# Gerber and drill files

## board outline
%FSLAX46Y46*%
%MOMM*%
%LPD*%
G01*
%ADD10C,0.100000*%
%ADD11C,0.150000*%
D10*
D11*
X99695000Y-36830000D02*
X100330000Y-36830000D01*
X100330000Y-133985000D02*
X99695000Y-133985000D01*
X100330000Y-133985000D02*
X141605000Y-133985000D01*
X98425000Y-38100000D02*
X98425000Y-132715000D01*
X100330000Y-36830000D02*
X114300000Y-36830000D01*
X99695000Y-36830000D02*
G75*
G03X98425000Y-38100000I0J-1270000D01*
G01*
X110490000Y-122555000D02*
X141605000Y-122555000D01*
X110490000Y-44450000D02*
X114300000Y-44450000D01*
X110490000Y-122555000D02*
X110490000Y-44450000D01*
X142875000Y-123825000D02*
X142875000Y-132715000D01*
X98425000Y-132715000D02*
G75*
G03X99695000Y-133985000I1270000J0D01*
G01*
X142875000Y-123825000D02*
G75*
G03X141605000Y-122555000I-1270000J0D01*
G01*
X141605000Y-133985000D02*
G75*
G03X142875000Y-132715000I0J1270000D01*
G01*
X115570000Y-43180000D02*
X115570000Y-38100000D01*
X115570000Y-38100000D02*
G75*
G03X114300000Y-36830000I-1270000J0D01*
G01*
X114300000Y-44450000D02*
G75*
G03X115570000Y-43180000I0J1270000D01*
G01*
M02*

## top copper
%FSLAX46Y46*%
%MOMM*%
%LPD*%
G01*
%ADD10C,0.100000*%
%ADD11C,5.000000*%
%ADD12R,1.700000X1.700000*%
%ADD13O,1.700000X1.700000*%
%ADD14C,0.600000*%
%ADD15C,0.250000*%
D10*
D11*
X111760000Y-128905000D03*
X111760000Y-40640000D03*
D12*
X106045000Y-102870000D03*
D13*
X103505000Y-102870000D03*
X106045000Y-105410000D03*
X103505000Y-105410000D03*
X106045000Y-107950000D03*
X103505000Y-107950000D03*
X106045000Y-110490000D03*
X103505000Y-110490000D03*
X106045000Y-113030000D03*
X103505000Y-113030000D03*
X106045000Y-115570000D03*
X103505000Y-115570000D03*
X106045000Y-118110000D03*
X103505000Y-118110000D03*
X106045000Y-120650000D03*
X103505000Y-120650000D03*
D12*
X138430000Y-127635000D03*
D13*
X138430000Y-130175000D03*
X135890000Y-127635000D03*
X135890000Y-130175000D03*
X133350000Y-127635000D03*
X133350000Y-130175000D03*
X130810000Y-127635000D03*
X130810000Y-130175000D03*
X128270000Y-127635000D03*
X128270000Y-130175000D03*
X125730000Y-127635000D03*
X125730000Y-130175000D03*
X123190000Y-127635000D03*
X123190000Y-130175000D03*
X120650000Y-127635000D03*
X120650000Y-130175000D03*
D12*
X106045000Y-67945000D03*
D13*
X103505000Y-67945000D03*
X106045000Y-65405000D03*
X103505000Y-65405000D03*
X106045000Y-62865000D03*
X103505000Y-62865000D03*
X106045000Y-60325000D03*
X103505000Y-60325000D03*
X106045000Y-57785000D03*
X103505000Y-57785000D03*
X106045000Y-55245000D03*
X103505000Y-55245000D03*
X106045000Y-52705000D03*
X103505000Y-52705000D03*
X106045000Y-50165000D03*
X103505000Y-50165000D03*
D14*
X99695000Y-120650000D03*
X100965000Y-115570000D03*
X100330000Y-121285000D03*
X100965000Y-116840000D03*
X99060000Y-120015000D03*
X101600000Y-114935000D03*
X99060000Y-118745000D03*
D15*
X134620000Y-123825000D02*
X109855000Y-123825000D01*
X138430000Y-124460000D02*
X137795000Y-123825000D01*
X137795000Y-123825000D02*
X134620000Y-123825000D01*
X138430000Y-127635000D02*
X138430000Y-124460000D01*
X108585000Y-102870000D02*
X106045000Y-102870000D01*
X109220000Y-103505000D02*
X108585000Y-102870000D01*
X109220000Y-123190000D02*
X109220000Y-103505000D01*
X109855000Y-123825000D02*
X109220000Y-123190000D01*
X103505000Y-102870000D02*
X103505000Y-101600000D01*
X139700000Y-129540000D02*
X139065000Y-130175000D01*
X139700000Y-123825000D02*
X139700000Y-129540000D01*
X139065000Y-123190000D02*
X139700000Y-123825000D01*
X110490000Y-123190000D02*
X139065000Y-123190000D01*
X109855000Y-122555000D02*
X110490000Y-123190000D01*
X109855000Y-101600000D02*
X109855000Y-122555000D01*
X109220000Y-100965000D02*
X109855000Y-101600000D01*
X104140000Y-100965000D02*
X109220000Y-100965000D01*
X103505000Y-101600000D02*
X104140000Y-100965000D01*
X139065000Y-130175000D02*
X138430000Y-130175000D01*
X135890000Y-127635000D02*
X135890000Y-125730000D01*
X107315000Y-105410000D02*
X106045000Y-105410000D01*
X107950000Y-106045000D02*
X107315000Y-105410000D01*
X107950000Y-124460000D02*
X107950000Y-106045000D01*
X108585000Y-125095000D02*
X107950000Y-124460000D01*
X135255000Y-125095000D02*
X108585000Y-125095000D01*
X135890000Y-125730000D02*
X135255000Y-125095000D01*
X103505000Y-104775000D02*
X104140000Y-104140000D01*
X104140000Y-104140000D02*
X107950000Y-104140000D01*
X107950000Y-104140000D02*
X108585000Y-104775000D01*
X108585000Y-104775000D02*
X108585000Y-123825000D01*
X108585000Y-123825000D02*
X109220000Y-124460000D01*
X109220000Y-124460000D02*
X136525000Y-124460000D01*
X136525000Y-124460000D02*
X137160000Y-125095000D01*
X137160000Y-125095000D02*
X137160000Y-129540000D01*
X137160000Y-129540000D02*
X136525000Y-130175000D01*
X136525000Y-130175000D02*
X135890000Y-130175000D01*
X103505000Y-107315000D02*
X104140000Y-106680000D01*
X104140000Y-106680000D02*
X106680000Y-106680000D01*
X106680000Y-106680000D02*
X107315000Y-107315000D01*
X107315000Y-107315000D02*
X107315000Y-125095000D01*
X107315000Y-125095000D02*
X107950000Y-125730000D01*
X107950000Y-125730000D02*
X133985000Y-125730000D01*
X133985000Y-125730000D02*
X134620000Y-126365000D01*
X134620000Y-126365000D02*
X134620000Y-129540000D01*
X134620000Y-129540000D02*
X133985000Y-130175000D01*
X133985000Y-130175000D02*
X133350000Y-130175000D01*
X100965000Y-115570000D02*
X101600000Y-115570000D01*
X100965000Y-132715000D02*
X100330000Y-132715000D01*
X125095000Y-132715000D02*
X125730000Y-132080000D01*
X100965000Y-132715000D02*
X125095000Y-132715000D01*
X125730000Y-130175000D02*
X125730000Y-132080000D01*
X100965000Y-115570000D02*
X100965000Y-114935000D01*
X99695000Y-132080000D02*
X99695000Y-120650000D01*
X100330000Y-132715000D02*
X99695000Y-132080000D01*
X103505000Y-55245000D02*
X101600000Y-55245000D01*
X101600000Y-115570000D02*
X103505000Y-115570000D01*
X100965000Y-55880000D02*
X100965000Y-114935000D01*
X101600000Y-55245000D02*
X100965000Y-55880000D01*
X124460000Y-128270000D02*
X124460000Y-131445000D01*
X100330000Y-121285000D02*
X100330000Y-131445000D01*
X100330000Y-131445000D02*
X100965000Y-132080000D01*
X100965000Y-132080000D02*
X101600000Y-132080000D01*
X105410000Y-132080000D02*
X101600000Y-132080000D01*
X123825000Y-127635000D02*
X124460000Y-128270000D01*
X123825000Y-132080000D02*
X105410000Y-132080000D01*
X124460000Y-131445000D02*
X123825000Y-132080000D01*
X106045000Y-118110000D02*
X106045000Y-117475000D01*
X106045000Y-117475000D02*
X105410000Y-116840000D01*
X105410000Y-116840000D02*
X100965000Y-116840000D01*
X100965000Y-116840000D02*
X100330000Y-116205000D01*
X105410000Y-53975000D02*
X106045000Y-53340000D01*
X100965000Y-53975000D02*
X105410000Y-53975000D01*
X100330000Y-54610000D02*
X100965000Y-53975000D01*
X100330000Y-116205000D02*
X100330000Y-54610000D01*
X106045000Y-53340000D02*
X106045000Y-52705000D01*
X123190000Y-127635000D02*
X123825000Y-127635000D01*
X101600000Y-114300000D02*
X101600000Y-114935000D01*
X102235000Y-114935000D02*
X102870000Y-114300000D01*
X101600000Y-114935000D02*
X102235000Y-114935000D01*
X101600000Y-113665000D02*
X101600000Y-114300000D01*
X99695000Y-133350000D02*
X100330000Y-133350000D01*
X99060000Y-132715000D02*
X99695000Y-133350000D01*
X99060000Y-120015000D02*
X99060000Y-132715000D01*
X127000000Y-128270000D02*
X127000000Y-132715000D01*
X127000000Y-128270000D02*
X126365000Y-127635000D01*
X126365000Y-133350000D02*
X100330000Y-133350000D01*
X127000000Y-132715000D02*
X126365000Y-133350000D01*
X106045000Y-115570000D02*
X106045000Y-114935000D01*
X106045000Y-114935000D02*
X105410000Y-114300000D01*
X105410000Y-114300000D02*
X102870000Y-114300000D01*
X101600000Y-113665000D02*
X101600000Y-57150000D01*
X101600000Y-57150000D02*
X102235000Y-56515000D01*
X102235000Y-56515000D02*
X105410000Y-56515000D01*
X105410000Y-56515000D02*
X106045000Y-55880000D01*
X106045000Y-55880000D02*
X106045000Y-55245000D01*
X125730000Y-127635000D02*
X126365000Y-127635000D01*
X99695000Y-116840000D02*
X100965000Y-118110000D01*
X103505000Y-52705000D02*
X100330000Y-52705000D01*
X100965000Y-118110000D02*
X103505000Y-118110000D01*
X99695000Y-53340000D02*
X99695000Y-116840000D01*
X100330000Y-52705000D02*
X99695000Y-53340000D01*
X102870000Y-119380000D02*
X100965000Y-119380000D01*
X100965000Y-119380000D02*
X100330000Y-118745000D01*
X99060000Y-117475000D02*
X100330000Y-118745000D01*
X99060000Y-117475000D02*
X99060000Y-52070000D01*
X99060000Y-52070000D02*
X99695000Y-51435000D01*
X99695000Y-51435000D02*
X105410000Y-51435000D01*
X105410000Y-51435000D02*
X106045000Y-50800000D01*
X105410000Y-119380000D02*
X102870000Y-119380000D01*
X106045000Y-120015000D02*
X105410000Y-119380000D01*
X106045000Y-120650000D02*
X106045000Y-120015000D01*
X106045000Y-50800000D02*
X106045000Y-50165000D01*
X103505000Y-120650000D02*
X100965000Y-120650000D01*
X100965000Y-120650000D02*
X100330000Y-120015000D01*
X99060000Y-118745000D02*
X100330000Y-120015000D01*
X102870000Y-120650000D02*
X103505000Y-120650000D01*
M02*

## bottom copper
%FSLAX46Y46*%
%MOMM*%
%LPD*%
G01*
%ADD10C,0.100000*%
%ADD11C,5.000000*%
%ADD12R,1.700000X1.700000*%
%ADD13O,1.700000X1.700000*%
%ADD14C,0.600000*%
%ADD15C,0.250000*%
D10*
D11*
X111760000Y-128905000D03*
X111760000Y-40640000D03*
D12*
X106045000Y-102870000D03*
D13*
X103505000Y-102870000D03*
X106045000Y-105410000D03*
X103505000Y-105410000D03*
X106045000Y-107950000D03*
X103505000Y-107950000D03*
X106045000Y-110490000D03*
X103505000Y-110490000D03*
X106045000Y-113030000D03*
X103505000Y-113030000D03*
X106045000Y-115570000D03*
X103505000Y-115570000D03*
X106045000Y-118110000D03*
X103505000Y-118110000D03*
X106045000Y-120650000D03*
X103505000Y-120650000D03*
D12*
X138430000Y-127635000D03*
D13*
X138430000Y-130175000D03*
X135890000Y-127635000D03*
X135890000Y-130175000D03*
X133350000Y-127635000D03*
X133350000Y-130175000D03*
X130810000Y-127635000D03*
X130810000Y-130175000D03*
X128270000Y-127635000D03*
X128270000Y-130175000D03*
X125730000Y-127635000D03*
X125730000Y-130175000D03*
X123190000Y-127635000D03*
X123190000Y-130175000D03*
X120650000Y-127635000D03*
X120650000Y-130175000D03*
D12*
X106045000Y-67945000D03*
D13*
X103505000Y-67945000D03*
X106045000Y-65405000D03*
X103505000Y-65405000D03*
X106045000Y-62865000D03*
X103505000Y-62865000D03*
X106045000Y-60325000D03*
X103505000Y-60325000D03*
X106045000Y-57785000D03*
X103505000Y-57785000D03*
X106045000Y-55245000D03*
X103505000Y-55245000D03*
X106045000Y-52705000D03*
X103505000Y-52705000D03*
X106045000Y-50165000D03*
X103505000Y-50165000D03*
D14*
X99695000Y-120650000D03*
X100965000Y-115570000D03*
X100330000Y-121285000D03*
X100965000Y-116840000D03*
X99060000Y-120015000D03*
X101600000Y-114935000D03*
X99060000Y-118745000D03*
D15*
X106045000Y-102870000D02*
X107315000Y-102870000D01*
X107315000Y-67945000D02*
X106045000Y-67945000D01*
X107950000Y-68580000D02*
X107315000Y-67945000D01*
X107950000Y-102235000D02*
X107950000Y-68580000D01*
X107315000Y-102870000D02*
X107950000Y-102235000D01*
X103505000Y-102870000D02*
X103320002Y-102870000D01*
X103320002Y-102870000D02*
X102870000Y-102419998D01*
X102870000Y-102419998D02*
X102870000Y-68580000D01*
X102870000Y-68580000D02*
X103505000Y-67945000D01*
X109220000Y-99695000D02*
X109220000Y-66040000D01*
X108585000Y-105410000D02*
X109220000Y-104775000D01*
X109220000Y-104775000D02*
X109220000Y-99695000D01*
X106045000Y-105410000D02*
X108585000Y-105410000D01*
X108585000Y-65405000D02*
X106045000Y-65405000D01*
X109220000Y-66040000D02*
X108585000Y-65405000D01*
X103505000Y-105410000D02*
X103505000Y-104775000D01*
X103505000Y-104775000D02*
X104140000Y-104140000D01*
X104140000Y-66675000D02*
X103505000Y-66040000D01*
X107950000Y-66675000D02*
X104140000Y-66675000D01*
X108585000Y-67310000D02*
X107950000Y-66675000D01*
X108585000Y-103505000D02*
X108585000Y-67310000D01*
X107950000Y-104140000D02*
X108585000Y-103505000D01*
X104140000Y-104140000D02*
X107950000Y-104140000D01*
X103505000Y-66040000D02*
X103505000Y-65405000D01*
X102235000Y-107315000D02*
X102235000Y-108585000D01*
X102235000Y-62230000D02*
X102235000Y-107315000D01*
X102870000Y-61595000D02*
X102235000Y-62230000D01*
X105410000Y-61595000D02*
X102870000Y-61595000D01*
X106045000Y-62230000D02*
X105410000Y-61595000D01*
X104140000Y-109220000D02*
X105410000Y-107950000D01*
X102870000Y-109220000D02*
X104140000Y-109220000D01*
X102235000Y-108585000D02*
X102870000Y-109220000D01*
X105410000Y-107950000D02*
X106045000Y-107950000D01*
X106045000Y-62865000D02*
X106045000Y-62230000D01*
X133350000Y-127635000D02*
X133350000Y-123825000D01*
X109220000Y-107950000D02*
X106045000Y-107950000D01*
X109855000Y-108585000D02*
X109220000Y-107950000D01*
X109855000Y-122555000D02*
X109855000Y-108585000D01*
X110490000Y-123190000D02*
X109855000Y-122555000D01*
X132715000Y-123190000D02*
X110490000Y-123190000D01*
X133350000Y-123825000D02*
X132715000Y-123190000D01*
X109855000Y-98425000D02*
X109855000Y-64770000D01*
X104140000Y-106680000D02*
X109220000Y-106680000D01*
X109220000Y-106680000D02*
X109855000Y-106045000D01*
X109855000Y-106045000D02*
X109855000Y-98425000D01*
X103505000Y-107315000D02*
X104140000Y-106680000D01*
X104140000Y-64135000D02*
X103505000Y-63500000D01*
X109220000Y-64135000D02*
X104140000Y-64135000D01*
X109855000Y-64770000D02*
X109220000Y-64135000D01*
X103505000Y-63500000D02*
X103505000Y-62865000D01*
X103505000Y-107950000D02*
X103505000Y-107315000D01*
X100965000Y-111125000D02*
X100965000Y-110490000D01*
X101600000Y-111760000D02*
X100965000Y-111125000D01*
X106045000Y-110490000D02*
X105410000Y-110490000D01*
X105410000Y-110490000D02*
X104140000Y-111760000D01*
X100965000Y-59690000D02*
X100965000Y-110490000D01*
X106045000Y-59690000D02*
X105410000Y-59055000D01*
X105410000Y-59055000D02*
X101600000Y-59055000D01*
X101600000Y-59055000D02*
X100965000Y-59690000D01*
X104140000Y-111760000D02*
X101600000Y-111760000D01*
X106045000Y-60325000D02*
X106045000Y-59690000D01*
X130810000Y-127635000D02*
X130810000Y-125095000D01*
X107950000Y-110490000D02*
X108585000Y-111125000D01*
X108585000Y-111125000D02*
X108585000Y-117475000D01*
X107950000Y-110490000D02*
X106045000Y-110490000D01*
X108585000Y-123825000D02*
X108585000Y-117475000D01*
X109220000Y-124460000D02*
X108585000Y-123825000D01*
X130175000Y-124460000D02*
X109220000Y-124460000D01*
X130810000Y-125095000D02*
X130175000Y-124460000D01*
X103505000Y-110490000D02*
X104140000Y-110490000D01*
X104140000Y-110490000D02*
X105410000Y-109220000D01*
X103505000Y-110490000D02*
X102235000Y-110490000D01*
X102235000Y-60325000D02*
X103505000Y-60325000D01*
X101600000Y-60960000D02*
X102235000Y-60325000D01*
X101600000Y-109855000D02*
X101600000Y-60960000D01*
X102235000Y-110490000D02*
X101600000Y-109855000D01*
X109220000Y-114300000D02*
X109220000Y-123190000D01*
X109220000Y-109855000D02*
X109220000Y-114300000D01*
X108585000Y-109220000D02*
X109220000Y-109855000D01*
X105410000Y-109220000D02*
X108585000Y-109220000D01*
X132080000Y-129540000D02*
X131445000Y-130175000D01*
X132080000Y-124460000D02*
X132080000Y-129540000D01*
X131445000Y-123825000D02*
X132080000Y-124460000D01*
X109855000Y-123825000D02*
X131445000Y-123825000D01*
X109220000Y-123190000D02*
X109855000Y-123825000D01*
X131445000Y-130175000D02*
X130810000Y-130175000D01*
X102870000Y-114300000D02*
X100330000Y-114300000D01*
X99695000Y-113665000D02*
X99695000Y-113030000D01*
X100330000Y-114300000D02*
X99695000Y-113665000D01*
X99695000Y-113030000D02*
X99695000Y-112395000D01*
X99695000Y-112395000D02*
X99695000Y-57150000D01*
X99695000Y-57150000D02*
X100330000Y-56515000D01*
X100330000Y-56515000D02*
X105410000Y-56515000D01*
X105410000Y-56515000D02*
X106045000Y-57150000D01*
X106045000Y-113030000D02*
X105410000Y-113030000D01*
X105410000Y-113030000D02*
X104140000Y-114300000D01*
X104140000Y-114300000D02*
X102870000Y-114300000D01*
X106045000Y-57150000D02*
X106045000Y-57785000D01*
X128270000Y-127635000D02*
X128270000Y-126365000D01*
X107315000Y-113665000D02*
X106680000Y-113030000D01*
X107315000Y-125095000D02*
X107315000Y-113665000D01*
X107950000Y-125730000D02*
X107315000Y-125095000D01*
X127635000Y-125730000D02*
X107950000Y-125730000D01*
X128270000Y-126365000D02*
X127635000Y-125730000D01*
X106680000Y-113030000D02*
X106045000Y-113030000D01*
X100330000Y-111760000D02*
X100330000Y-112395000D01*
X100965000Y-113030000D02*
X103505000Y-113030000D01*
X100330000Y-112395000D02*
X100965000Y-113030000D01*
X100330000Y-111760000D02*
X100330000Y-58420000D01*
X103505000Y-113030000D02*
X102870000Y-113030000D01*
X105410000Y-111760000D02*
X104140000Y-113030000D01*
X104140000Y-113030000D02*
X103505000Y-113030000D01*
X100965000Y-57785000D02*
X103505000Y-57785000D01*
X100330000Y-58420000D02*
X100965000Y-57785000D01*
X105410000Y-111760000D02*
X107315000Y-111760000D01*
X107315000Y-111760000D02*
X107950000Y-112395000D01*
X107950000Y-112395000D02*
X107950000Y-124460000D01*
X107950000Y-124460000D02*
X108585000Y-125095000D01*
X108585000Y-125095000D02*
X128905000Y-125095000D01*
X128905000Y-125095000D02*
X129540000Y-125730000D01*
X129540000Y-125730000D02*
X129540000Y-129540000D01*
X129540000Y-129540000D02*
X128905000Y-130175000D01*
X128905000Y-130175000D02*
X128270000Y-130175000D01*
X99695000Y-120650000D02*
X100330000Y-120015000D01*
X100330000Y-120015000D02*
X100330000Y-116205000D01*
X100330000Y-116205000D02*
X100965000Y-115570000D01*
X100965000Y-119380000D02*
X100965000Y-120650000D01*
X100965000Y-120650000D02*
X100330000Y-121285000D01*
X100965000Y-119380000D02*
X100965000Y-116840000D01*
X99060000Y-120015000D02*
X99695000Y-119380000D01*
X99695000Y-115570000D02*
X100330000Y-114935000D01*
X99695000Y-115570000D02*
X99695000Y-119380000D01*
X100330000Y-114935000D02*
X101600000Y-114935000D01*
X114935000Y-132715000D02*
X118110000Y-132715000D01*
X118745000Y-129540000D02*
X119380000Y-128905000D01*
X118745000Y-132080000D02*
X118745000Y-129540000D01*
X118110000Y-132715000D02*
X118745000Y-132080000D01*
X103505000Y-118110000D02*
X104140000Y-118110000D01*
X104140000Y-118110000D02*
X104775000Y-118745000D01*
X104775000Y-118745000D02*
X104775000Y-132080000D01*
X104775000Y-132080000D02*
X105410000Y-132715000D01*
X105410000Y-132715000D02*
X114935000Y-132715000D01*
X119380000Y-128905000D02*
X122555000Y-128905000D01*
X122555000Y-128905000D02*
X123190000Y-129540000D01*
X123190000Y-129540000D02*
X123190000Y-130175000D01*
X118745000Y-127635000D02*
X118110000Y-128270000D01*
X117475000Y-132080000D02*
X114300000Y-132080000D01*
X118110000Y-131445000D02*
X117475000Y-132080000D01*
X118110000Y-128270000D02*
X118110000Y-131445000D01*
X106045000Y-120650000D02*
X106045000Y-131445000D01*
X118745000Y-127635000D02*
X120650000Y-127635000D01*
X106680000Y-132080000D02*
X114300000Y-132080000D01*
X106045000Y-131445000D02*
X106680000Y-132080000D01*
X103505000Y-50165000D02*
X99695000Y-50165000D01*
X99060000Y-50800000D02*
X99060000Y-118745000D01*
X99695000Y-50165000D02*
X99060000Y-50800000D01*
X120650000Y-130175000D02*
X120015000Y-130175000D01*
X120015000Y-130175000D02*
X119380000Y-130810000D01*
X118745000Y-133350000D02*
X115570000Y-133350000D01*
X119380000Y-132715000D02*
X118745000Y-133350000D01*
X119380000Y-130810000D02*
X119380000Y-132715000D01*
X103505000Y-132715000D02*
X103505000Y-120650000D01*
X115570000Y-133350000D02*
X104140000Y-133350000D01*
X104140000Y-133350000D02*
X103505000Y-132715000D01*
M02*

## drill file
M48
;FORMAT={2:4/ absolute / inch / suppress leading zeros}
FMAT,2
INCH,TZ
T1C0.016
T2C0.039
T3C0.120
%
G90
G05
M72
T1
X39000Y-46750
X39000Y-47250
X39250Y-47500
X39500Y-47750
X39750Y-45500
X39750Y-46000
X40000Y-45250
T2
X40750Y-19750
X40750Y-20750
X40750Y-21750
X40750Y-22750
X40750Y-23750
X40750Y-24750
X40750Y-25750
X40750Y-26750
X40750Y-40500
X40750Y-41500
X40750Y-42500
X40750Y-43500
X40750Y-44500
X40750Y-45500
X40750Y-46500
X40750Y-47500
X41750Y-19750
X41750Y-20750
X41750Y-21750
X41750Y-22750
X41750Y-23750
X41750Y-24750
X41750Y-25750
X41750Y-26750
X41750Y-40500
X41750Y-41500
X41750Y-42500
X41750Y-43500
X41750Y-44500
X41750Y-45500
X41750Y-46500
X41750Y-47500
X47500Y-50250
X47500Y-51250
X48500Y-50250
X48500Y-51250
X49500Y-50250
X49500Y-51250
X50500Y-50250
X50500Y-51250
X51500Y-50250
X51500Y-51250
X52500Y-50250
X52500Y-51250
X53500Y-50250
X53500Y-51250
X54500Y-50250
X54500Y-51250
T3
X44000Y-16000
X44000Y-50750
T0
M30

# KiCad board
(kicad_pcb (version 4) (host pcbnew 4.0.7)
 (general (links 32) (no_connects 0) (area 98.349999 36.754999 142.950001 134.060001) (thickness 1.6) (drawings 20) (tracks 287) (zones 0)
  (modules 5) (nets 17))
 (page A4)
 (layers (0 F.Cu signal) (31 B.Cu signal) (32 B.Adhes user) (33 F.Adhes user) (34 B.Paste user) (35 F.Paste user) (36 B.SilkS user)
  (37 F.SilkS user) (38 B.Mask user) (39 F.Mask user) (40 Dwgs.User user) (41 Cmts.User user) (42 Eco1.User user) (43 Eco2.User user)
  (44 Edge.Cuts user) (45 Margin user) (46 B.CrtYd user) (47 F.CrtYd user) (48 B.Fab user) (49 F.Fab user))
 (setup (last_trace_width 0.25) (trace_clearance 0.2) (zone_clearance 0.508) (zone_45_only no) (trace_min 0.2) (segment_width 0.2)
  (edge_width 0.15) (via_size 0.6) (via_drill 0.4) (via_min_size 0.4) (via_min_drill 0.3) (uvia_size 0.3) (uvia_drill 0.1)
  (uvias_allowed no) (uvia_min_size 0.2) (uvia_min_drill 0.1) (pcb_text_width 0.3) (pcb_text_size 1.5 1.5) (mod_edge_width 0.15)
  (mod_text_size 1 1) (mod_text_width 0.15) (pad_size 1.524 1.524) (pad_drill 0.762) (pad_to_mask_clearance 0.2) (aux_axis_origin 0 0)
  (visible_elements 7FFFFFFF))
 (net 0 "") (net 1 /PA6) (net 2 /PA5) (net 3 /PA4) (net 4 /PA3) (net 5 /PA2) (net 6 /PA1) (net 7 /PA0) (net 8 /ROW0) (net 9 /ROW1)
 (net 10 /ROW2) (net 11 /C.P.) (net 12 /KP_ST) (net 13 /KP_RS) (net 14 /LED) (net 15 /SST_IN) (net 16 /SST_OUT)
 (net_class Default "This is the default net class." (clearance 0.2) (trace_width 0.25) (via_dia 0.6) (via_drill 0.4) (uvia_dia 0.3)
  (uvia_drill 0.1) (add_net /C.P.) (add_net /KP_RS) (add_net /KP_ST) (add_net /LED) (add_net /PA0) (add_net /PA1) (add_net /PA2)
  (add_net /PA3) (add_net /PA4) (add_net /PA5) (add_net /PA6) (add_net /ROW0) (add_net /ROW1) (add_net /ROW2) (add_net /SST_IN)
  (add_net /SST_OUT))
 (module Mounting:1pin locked (layer F.Cu) (at 111.76 128.905)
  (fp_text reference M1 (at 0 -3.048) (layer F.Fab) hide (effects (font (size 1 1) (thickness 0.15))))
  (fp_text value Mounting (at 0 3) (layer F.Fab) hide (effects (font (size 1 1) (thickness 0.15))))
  (pad 1 thru_hole circle (at 0 0) (size 5 5) (drill 3.048) (layers *.Cu *.Mask)))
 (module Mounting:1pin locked (layer F.Cu) (at 111.76 40.64)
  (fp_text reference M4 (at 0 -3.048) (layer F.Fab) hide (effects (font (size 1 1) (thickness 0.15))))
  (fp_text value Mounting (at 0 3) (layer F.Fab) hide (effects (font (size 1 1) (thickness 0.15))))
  (pad 1 thru_hole circle (at 0 0) (size 5 5) (drill 3.048) (layers *.Cu *.Mask)))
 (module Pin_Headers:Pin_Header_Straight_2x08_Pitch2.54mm (layer B.Cu) (at 106.045 102.87 180)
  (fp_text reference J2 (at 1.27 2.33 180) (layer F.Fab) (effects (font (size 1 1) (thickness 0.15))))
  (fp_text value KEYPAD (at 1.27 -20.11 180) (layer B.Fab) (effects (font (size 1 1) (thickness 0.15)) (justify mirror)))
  (pad 1 thru_hole rect (at 0 0 180) (size 1.7 1.7) (drill 1) (layers *.Cu *.Mask) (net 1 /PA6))
  (pad 2 thru_hole oval (at 2.54 0 180) (size 1.7 1.7) (drill 1) (layers *.Cu *.Mask) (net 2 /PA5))
  (pad 3 thru_hole oval (at 0 -2.54 180) (size 1.7 1.7) (drill 1) (layers *.Cu *.Mask) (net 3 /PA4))
  (pad 4 thru_hole oval (at 2.54 -2.54 180) (size 1.7 1.7) (drill 1) (layers *.Cu *.Mask) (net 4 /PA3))
  (pad 5 thru_hole oval (at 0 -5.08 180) (size 1.7 1.7) (drill 1) (layers *.Cu *.Mask) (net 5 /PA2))
  (pad 6 thru_hole oval (at 2.54 -5.08 180) (size 1.7 1.7) (drill 1) (layers *.Cu *.Mask) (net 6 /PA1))
  (pad 7 thru_hole oval (at 0 -7.62 180) (size 1.7 1.7) (drill 1) (layers *.Cu *.Mask) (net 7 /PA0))
  (pad 8 thru_hole oval (at 2.54 -7.62 180) (size 1.7 1.7) (drill 1) (layers *.Cu *.Mask) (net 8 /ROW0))
  (pad 9 thru_hole oval (at 0 -10.16 180) (size 1.7 1.7) (drill 1) (layers *.Cu *.Mask) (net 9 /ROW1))
  (pad 10 thru_hole oval (at 2.54 -10.16 180) (size 1.7 1.7) (drill 1) (layers *.Cu *.Mask) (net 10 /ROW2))
  (pad 11 thru_hole oval (at 0 -12.7 180) (size 1.7 1.7) (drill 1) (layers *.Cu *.Mask) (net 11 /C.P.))
  (pad 12 thru_hole oval (at 2.54 -12.7 180) (size 1.7 1.7) (drill 1) (layers *.Cu *.Mask) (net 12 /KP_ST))
  (pad 13 thru_hole oval (at 0 -15.24 180) (size 1.7 1.7) (drill 1) (layers *.Cu *.Mask) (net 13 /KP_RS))
  (pad 14 thru_hole oval (at 2.54 -15.24 180) (size 1.7 1.7) (drill 1) (layers *.Cu *.Mask) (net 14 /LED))
  (pad 15 thru_hole oval (at 0 -17.78 180) (size 1.7 1.7) (drill 1) (layers *.Cu *.Mask) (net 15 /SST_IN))
  (pad 16 thru_hole oval (at 2.54 -17.78 180) (size 1.7 1.7) (drill 1) (layers *.Cu *.Mask) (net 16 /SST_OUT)))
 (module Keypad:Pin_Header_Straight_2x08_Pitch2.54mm (layer F.Cu) (at 138.43 127.635 270)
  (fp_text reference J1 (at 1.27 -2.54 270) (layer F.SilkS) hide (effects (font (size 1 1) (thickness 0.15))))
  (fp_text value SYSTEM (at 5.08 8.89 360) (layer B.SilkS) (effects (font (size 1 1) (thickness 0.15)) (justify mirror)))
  (pad 1 thru_hole rect (at 0 0 270) (size 1.7 1.7) (drill 1) (layers *.Cu *.Mask) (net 1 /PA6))
  (pad 2 thru_hole oval (at 2.54 0 270) (size 1.7 1.7) (drill 1) (layers *.Cu *.Mask) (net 2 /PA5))
  (pad 3 thru_hole oval (at 0 2.54 270) (size 1.7 1.7) (drill 1) (layers *.Cu *.Mask) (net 3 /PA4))
  (pad 4 thru_hole oval (at 2.54 2.54 270) (size 1.7 1.7) (drill 1) (layers *.Cu *.Mask) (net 4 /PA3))
  (pad 5 thru_hole oval (at 0 5.08 270) (size 1.7 1.7) (drill 1) (layers *.Cu *.Mask) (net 5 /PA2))
  (pad 6 thru_hole oval (at 2.54 5.08 270) (size 1.7 1.7) (drill 1) (layers *.Cu *.Mask) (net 6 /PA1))
  (pad 7 thru_hole oval (at 0 7.62 270) (size 1.7 1.7) (drill 1) (layers *.Cu *.Mask) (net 7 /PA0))
  (pad 8 thru_hole oval (at 2.54 7.62 270) (size 1.7 1.7) (drill 1) (layers *.Cu *.Mask) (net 8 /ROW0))
  (pad 9 thru_hole oval (at 0 10.16 270) (size 1.7 1.7) (drill 1) (layers *.Cu *.Mask) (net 9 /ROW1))
  (pad 10 thru_hole oval (at 2.54 10.16 270) (size 1.7 1.7) (drill 1) (layers *.Cu *.Mask) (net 10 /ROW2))
  (pad 11 thru_hole oval (at 0 12.7 270) (size 1.7 1.7) (drill 1) (layers *.Cu *.Mask) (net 11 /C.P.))
  (pad 12 thru_hole oval (at 2.54 12.7 270) (size 1.7 1.7) (drill 1) (layers *.Cu *.Mask) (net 12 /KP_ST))
  (pad 13 thru_hole oval (at 0 15.24 270) (size 1.7 1.7) (drill 1) (layers *.Cu *.Mask) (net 13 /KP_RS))
  (pad 14 thru_hole oval (at 2.54 15.24 270) (size 1.7 1.7) (drill 1) (layers *.Cu *.Mask) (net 14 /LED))
  (pad 15 thru_hole oval (at 0 17.78 270) (size 1.7 1.7) (drill 1) (layers *.Cu *.Mask) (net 15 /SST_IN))
  (pad 16 thru_hole oval (at 2.54 17.78 270) (size 1.7 1.7) (drill 1) (layers *.Cu *.Mask) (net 16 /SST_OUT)))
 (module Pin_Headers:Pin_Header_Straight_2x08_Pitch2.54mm (layer F.Cu) (at 106.045 67.945 180)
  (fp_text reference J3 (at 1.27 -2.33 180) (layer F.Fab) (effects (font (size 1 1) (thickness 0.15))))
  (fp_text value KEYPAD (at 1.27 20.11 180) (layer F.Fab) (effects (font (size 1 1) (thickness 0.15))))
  (pad 1 thru_hole rect (at 0 0 180) (size 1.7 1.7) (drill 1) (layers *.Cu *.Mask) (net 1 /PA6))
  (pad 2 thru_hole oval (at 2.54 0 180) (size 1.7 1.7) (drill 1) (layers *.Cu *.Mask) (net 2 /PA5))
  (pad 3 thru_hole oval (at 0 2.54 180) (size 1.7 1.7) (drill 1) (layers *.Cu *.Mask) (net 3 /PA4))
  (pad 4 thru_hole oval (at 2.54 2.54 180) (size 1.7 1.7) (drill 1) (layers *.Cu *.Mask) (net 4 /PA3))
  (pad 5 thru_hole oval (at 0 5.08 180) (size 1.7 1.7) (drill 1) (layers *.Cu *.Mask) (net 5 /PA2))
  (pad 6 thru_hole oval (at 2.54 5.08 180) (size 1.7 1.7) (drill 1) (layers *.Cu *.Mask) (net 6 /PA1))
  (pad 7 thru_hole oval (at 0 7.62 180) (size 1.7 1.7) (drill 1) (layers *.Cu *.Mask) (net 7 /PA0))
  (pad 8 thru_hole oval (at 2.54 7.62 180) (size 1.7 1.7) (drill 1) (layers *.Cu *.Mask) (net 8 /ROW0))
  (pad 9 thru_hole oval (at 0 10.16 180) (size 1.7 1.7) (drill 1) (layers *.Cu *.Mask) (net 9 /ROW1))
  (pad 10 thru_hole oval (at 2.54 10.16 180) (size 1.7 1.7) (drill 1) (layers *.Cu *.Mask) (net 10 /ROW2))
  (pad 11 thru_hole oval (at 0 12.7 180) (size 1.7 1.7) (drill 1) (layers *.Cu *.Mask) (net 11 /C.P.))
  (pad 12 thru_hole oval (at 2.54 12.7 180) (size 1.7 1.7) (drill 1) (layers *.Cu *.Mask) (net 12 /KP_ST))
  (pad 13 thru_hole oval (at 0 15.24 180) (size 1.7 1.7) (drill 1) (layers *.Cu *.Mask) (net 13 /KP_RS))
  (pad 14 thru_hole oval (at 2.54 15.24 180) (size 1.7 1.7) (drill 1) (layers *.Cu *.Mask) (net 14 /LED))
  (pad 15 thru_hole oval (at 0 17.78 180) (size 1.7 1.7) (drill 1) (layers *.Cu *.Mask) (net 15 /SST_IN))
  (pad 16 thru_hole oval (at 2.54 17.78 180) (size 1.7 1.7) (drill 1) (layers *.Cu *.Mask) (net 16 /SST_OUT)))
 (gr_line (start 99.695 36.83) (end 100.33 36.83) (angle 90) (layer Edge.Cuts) (width 0.15))
 (gr_line (start 100.33 133.985) (end 99.695 133.985) (angle 90) (layer Edge.Cuts) (width 0.15))
 (gr_line (start 100.33 133.985) (end 141.605 133.985) (angle 90) (layer Edge.Cuts) (width 0.15))
 (gr_line (start 98.425 38.1) (end 98.425 132.715) (angle 90) (layer Edge.Cuts) (width 0.15))
 (gr_line (start 100.33 36.83) (end 114.3 36.83) (angle 90) (layer Edge.Cuts) (width 0.15))
 (gr_arc (start 99.695 38.1) (end 98.425 38.1) (angle 90) (layer Edge.Cuts) (width 0.15))
 (gr_line (start 110.49 122.555) (end 141.605 122.555) (angle 90) (layer Edge.Cuts) (width 0.15))
 (gr_line (start 110.49 44.45) (end 114.3 44.45) (angle 90) (layer Edge.Cuts) (width 0.15))
 (gr_line (start 110.49 122.555) (end 110.49 44.45) (angle 90) (layer Edge.Cuts) (width 0.15))
 (gr_line (start 142.875 123.825) (end 142.875 132.715) (angle 90) (layer Edge.Cuts) (width 0.15))
 (gr_arc (start 99.695 132.715) (end 99.695 133.985) (angle 90) (layer Edge.Cuts) (width 0.15))
 (gr_arc (start 141.605 123.825) (end 141.605 122.555) (angle 90) (layer Edge.Cuts) (width 0.15))
 (gr_arc (start 141.605 132.715) (end 142.875 132.715) (angle 90) (layer Edge.Cuts) (width 0.15))
 (gr_line (start 115.57 43.18) (end 115.57 38.1) (angle 90) (layer Edge.Cuts) (width 0.15))
 (gr_arc (start 114.3 38.1) (end 114.3 36.83) (angle 90) (layer Edge.Cuts) (width 0.15))
 (gr_arc (start 114.3 43.18) (end 115.57 43.18) (angle 90) (layer Edge.Cuts) (width 0.15))
 (segment (start 106.045 102.87) (end 107.315 102.87) (width 0.25) (layer B.Cu) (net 1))
 (segment (start 107.315 67.945) (end 106.045 67.945) (width 0.25) (layer B.Cu) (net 1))
 (segment (start 107.95 68.58) (end 107.315 67.945) (width 0.25) (layer B.Cu) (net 1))
 (segment (start 107.95 102.235) (end 107.95 68.58) (width 0.25) (layer B.Cu) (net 1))
 (segment (start 107.315 102.87) (end 107.95 102.235) (width 0.25) (layer B.Cu) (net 1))
 (segment (start 134.62 123.825) (end 109.855 123.825) (width 0.25) (layer F.Cu) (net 1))
 (segment (start 138.43 124.46) (end 137.795 123.825) (width 0.25) (layer F.Cu) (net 1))
 (segment (start 137.795 123.825) (end 134.62 123.825) (width 0.25) (layer F.Cu) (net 1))
 (segment (start 138.43 127.635) (end 138.43 124.46) (width 0.25) (layer F.Cu) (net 1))
 (segment (start 108.585 102.87) (end 106.045 102.87) (width 0.25) (layer F.Cu) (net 1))
 (segment (start 109.22 103.505) (end 108.585 102.87) (width 0.25) (layer F.Cu) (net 1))
 (segment (start 109.22 123.19) (end 109.22 103.505) (width 0.25) (layer F.Cu) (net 1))
 (segment (start 109.855 123.825) (end 109.22 123.19) (width 0.25) (layer F.Cu) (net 1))
 (segment (start 103.505 102.87) (end 103.320002 102.87) (width 0.25) (layer B.Cu) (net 2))
 (segment (start 103.320002 102.87) (end 102.87 102.419998) (width 0.25) (layer B.Cu) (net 2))
 (segment (start 102.87 102.419998) (end 102.87 68.58) (width 0.25) (layer B.Cu) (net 2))
 (segment (start 102.87 68.58) (end 103.505 67.945) (width 0.25) (layer B.Cu) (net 2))
 (segment (start 103.505 102.87) (end 103.505 101.6) (width 0.25) (layer F.Cu) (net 2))
 (segment (start 139.7 129.54) (end 139.065 130.175) (width 0.25) (layer F.Cu) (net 2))
 (segment (start 139.7 123.825) (end 139.7 129.54) (width 0.25) (layer F.Cu) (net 2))
 (segment (start 139.065 123.19) (end 139.7 123.825) (width 0.25) (layer F.Cu) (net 2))
 (segment (start 110.49 123.19) (end 139.065 123.19) (width 0.25) (layer F.Cu) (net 2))
 (segment (start 109.855 122.555) (end 110.49 123.19) (width 0.25) (layer F.Cu) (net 2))
 (segment (start 109.855 101.6) (end 109.855 122.555) (width 0.25) (layer F.Cu) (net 2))
 (segment (start 109.22 100.965) (end 109.855 101.6) (width 0.25) (layer F.Cu) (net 2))
 (segment (start 104.14 100.965) (end 109.22 100.965) (width 0.25) (layer F.Cu) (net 2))
 (segment (start 103.505 101.6) (end 104.14 100.965) (width 0.25) (layer F.Cu) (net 2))
 (segment (start 139.065 130.175) (end 138.43 130.175) (width 0.25) (layer F.Cu) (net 2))
 (segment (start 109.22 99.695) (end 109.22 66.04) (width 0.25) (layer B.Cu) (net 3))
 (segment (start 108.585 105.41) (end 109.22 104.775) (width 0.25) (layer B.Cu) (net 3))
 (segment (start 109.22 104.775) (end 109.22 99.695) (width 0.25) (layer B.Cu) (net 3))
 (segment (start 106.045 105.41) (end 108.585 105.41) (width 0.25) (layer B.Cu) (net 3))
 (segment (start 108.585 65.405) (end 106.045 65.405) (width 0.25) (layer B.Cu) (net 3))
 (segment (start 109.22 66.04) (end 108.585 65.405) (width 0.25) (layer B.Cu) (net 3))
 (segment (start 135.89 127.635) (end 135.89 125.73) (width 0.25) (layer F.Cu) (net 3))
 (segment (start 107.315 105.41) (end 106.045 105.41) (width 0.25) (layer F.Cu) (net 3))
 (segment (start 107.95 106.045) (end 107.315 105.41) (width 0.25) (layer F.Cu) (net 3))
 (segment (start 107.95 124.46) (end 107.95 106.045) (width 0.25) (layer F.Cu) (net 3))
 (segment (start 108.585 125.095) (end 107.95 124.46) (width 0.25) (layer F.Cu) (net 3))
 (segment (start 135.255 125.095) (end 108.585 125.095) (width 0.25) (layer F.Cu) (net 3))
 (segment (start 135.89 125.73) (end 135.255 125.095) (width 0.25) (layer F.Cu) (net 3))
 (segment (start 103.505 105.41) (end 103.505 104.775) (width 0.25) (layer B.Cu) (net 4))
 (segment (start 103.505 104.775) (end 104.14 104.14) (width 0.25) (layer B.Cu) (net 4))
 (segment (start 104.14 66.675) (end 103.505 66.04) (width 0.25) (layer B.Cu) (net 4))
 (segment (start 107.95 66.675) (end 104.14 66.675) (width 0.25) (layer B.Cu) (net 4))
 (segment (start 108.585 67.31) (end 107.95 66.675) (width 0.25) (layer B.Cu) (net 4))
 (segment (start 108.585 103.505) (end 108.585 67.31) (width 0.25) (layer B.Cu) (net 4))
 (segment (start 107.95 104.14) (end 108.585 103.505) (width 0.25) (layer B.Cu) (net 4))
 (segment (start 104.14 104.14) (end 107.95 104.14) (width 0.25) (layer B.Cu) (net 4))
 (segment (start 103.505 66.04) (end 103.505 65.405) (width 0.25) (layer B.Cu) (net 4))
 (segment (start 103.505 104.775) (end 104.14 104.14) (width 0.25) (layer F.Cu) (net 4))
 (segment (start 104.14 104.14) (end 107.95 104.14) (width 0.25) (layer F.Cu) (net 4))
 (segment (start 107.95 104.14) (end 108.585 104.775) (width 0.25) (layer F.Cu) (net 4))
 (segment (start 108.585 104.775) (end 108.585 123.825) (width 0.25) (layer F.Cu) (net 4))
 (segment (start 108.585 123.825) (end 109.22 124.46) (width 0.25) (layer F.Cu) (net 4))
 (segment (start 109.22 124.46) (end 136.525 124.46) (width 0.25) (layer F.Cu) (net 4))
 (segment (start 136.525 124.46) (end 137.16 125.095) (width 0.25) (layer F.Cu) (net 4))
 (segment (start 137.16 125.095) (end 137.16 129.54) (width 0.25) (layer F.Cu) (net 4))
 (segment (start 137.16 129.54) (end 136.525 130.175) (width 0.25) (layer F.Cu) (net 4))
 (segment (start 136.525 130.175) (end 135.89 130.175) (width 0.25) (layer F.Cu) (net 4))
 (segment (start 102.235 107.315) (end 102.235 108.585) (width 0.25) (layer B.Cu) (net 5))
 (segment (start 102.235 62.23) (end 102.235 107.315) (width 0.25) (layer B.Cu) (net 5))
 (segment (start 102.87 61.595) (end 102.235 62.23) (width 0.25) (layer B.Cu) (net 5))
 (segment (start 105.41 61.595) (end 102.87 61.595) (width 0.25) (layer B.Cu) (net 5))
 (segment (start 106.045 62.23) (end 105.41 61.595) (width 0.25) (layer B.Cu) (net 5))
 (segment (start 104.14 109.22) (end 105.41 107.95) (width 0.25) (layer B.Cu) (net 5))
 (segment (start 102.87 109.22) (end 104.14 109.22) (width 0.25) (layer B.Cu) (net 5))
 (segment (start 102.235 108.585) (end 102.87 109.22) (width 0.25) (layer B.Cu) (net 5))
 (segment (start 105.41 107.95) (end 106.045 107.95) (width 0.25) (layer B.Cu) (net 5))
 (segment (start 106.045 62.865) (end 106.045 62.23) (width 0.25) (layer B.Cu) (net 5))
 (segment (start 133.35 127.635) (end 133.35 123.825) (width 0.25) (layer B.Cu) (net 5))
 (segment (start 109.22 107.95) (end 106.045 107.95) (width 0.25) (layer B.Cu) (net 5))
 (segment (start 109.855 108.585) (end 109.22 107.95) (width 0.25) (layer B.Cu) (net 5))
 (segment (start 109.855 122.555) (end 109.855 108.585) (width 0.25) (layer B.Cu) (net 5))
 (segment (start 110.49 123.19) (end 109.855 122.555) (width 0.25) (layer B.Cu) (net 5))
 (segment (start 132.715 123.19) (end 110.49 123.19) (width 0.25) (layer B.Cu) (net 5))
 (segment (start 133.35 123.825) (end 132.715 123.19) (width 0.25) (layer B.Cu) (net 5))
 (segment (start 109.855 98.425) (end 109.855 64.77) (width 0.25) (layer B.Cu) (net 6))
 (segment (start 104.14 106.68) (end 109.22 106.68) (width 0.25) (layer B.Cu) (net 6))
 (segment (start 109.22 106.68) (end 109.855 106.045) (width 0.25) (layer B.Cu) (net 6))
 (segment (start 109.855 106.045) (end 109.855 98.425) (width 0.25) (layer B.Cu) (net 6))
 (segment (start 103.505 107.315) (end 104.14 106.68) (width 0.25) (layer B.Cu) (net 6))
 (segment (start 104.14 64.135) (end 103.505 63.5) (width 0.25) (layer B.Cu) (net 6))
 (segment (start 109.22 64.135) (end 104.14 64.135) (width 0.25) (layer B.Cu) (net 6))
 (segment (start 109.855 64.77) (end 109.22 64.135) (width 0.25) (layer B.Cu) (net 6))
 (segment (start 103.505 63.5) (end 103.505 62.865) (width 0.25) (layer B.Cu) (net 6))
 (segment (start 103.505 107.95) (end 103.505 107.315) (width 0.25) (layer B.Cu) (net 6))
 (segment (start 103.505 107.315) (end 104.14 106.68) (width 0.25) (layer F.Cu) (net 6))
 (segment (start 104.14 106.68) (end 106.68 106.68) (width 0.25) (layer F.Cu) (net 6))
 (segment (start 106.68 106.68) (end 107.315 107.315) (width 0.25) (layer F.Cu) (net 6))
 (segment (start 107.315 107.315) (end 107.315 125.095) (width 0.25) (layer F.Cu) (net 6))
 (segment (start 107.315 125.095) (end 107.95 125.73) (width 0.25) (layer F.Cu) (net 6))
 (segment (start 107.95 125.73) (end 133.985 125.73) (width 0.25) (layer F.Cu) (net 6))
 (segment (start 133.985 125.73) (end 134.62 126.365) (width 0.25) (layer F.Cu) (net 6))
 (segment (start 134.62 126.365) (end 134.62 129.54) (width 0.25) (layer F.Cu) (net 6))
 (segment (start 134.62 129.54) (end 133.985 130.175) (width 0.25) (layer F.Cu) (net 6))
 (segment (start 133.985 130.175) (end 133.35 130.175) (width 0.25) (layer F.Cu) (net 6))
 (segment (start 100.965 111.125) (end 100.965 110.49) (width 0.25) (layer B.Cu) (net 7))
 (segment (start 101.6 111.76) (end 100.965 111.125) (width 0.25) (layer B.Cu) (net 7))
 (segment (start 106.045 110.49) (end 105.41 110.49) (width 0.25) (layer B.Cu) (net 7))
 (segment (start 105.41 110.49) (end 104.14 111.76) (width 0.25) (layer B.Cu) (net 7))
 (segment (start 100.965 59.69) (end 100.965 110.49) (width 0.25) (layer B.Cu) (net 7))
 (segment (start 106.045 59.69) (end 105.41 59.055) (width 0.25) (layer B.Cu) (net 7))
 (segment (start 105.41 59.055) (end 101.6 59.055) (width 0.25) (layer B.Cu) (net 7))
 (segment (start 101.6 59.055) (end 100.965 59.69) (width 0.25) (layer B.Cu) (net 7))
 (segment (start 104.14 111.76) (end 101.6 111.76) (width 0.25) (layer B.Cu) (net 7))
 (segment (start 106.045 60.325) (end 106.045 59.69) (width 0.25) (layer B.Cu) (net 7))
 (segment (start 130.81 127.635) (end 130.81 125.095) (width 0.25) (layer B.Cu) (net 7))
 (segment (start 107.95 110.49) (end 108.585 111.125) (width 0.25) (layer B.Cu) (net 7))
 (segment (start 108.585 111.125) (end 108.585 117.475) (width 0.25) (layer B.Cu) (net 7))
 (segment (start 107.95 110.49) (end 106.045 110.49) (width 0.25) (layer B.Cu) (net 7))
 (segment (start 108.585 123.825) (end 108.585 117.475) (width 0.25) (layer B.Cu) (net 7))
 (segment (start 109.22 124.46) (end 108.585 123.825) (width 0.25) (layer B.Cu) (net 7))
 (segment (start 130.175 124.46) (end 109.22 124.46) (width 0.25) (layer B.Cu) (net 7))
 (segment (start 130.81 125.095) (end 130.175 124.46) (width 0.25) (layer B.Cu) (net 7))
 (segment (start 103.505 110.49) (end 104.14 110.49) (width 0.25) (layer B.Cu) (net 8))
 (segment (start 104.14 110.49) (end 105.41 109.22) (width 0.25) (layer B.Cu) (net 8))
 (segment (start 103.505 110.49) (end 102.235 110.49) (width 0.25) (layer B.Cu) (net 8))
 (segment (start 102.235 60.325) (end 103.505 60.325) (width 0.25) (layer B.Cu) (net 8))
 (segment (start 101.6 60.96) (end 102.235 60.325) (width 0.25) (layer B.Cu) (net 8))
 (segment (start 101.6 109.855) (end 101.6 60.96) (width 0.25) (layer B.Cu) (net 8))
 (segment (start 102.235 110.49) (end 101.6 109.855) (width 0.25) (layer B.Cu) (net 8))
 (segment (start 109.22 114.3) (end 109.22 123.19) (width 0.25) (layer B.Cu) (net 8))
 (segment (start 109.22 109.855) (end 109.22 114.3) (width 0.25) (layer B.Cu) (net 8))
 (segment (start 108.585 109.22) (end 109.22 109.855) (width 0.25) (layer B.Cu) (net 8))
 (segment (start 105.41 109.22) (end 108.585 109.22) (width 0.25) (layer B.Cu) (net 8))
 (segment (start 132.08 129.54) (end 131.445 130.175) (width 0.25) (layer B.Cu) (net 8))
 (segment (start 132.08 124.46) (end 132.08 129.54) (width 0.25) (layer B.Cu) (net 8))
 (segment (start 131.445 123.825) (end 132.08 124.46) (width 0.25) (layer B.Cu) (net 8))
 (segment (start 109.855 123.825) (end 131.445 123.825) (width 0.25) (layer B.Cu) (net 8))
 (segment (start 109.22 123.19) (end 109.855 123.825) (width 0.25) (layer B.Cu) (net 8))
 (segment (start 131.445 130.175) (end 130.81 130.175) (width 0.25) (layer B.Cu) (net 8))
 (segment (start 102.87 114.3) (end 100.33 114.3) (width 0.25) (layer B.Cu) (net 9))
 (segment (start 99.695 113.665) (end 99.695 113.03) (width 0.25) (layer B.Cu) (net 9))
 (segment (start 100.33 114.3) (end 99.695 113.665) (width 0.25) (layer B.Cu) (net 9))
 (segment (start 99.695 113.03) (end 99.695 112.395) (width 0.25) (layer B.Cu) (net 9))
 (segment (start 99.695 112.395) (end 99.695 57.15) (width 0.25) (layer B.Cu) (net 9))
 (segment (start 99.695 57.15) (end 100.33 56.515) (width 0.25) (layer B.Cu) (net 9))
 (segment (start 100.33 56.515) (end 105.41 56.515) (width 0.25) (layer B.Cu) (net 9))
 (segment (start 105.41 56.515) (end 106.045 57.15) (width 0.25) (layer B.Cu) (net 9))
 (segment (start 106.045 113.03) (end 105.41 113.03) (width 0.25) (layer B.Cu) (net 9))
 (segment (start 105.41 113.03) (end 104.14 114.3) (width 0.25) (layer B.Cu) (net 9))
 (segment (start 104.14 114.3) (end 102.87 114.3) (width 0.25) (layer B.Cu) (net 9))
 (segment (start 106.045 57.15) (end 106.045 57.785) (width 0.25) (layer B.Cu) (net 9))
 (segment (start 128.27 127.635) (end 128.27 126.365) (width 0.25) (layer B.Cu) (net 9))
 (segment (start 107.315 113.665) (end 106.68 113.03) (width 0.25) (layer B.Cu) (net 9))
 (segment (start 107.315 125.095) (end 107.315 113.665) (width 0.25) (layer B.Cu) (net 9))
 (segment (start 107.95 125.73) (end 107.315 125.095) (width 0.25) (layer B.Cu) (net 9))
 (segment (start 127.635 125.73) (end 107.95 125.73) (width 0.25) (layer B.Cu) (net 9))
 (segment (start 128.27 126.365) (end 127.635 125.73) (width 0.25) (layer B.Cu) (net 9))
 (segment (start 106.68 113.03) (end 106.045 113.03) (width 0.25) (layer B.Cu) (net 9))
 (segment (start 100.33 111.76) (end 100.33 112.395) (width 0.25) (layer B.Cu) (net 10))
 (segment (start 100.965 113.03) (end 103.505 113.03) (width 0.25) (layer B.Cu) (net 10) (status 800000))
 (segment (start 100.33 112.395) (end 100.965 113.03) (width 0.25) (layer B.Cu) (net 10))
 (segment (start 100.33 111.76) (end 100.33 58.42) (width 0.25) (layer B.Cu) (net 10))
 (segment (start 103.505 113.03) (end 102.87 113.03) (width 0.25) (layer B.Cu) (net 10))
 (segment (start 105.41 111.76) (end 104.14 113.03) (width 0.25) (layer B.Cu) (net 10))
 (segment (start 104.14 113.03) (end 103.505 113.03) (width 0.25) (layer B.Cu) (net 10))
 (segment (start 100.965 57.785) (end 103.505 57.785) (width 0.25) (layer B.Cu) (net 10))
 (segment (start 100.33 58.42) (end 100.965 57.785) (width 0.25) (layer B.Cu) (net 10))
 (segment (start 105.41 111.76) (end 107.315 111.76) (width 0.25) (layer B.Cu) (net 10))
 (segment (start 107.315 111.76) (end 107.95 112.395) (width 0.25) (layer B.Cu) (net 10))
 (segment (start 107.95 112.395) (end 107.95 124.46) (width 0.25) (layer B.Cu) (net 10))
 (segment (start 107.95 124.46) (end 108.585 125.095) (width 0.25) (layer B.Cu) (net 10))
 (segment (start 108.585 125.095) (end 128.905 125.095) (width 0.25) (layer B.Cu) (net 10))
 (segment (start 128.905 125.095) (end 129.54 125.73) (width 0.25) (layer B.Cu) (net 10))
 (segment (start 129.54 125.73) (end 129.54 129.54) (width 0.25) (layer B.Cu) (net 10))
 (segment (start 129.54 129.54) (end 128.905 130.175) (width 0.25) (layer B.Cu) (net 10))
 (segment (start 128.905 130.175) (end 128.27 130.175) (width 0.25) (layer B.Cu) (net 10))
 (via (at 99.695 120.65) (size 0.6) (drill 0.4) (layers F.Cu B.Cu) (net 12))
 (segment (start 99.695 120.65) (end 100.33 120.015) (width 0.25) (layer B.Cu) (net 12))
 (segment (start 100.965 115.57) (end 101.6 115.57) (width 0.25) (layer F.Cu) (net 12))
 (segment (start 100.965 132.715) (end 100.33 132.715) (width 0.25) (layer F.Cu) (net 12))
 (segment (start 125.095 132.715) (end 125.73 132.08) (width 0.25) (layer F.Cu) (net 12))
 (segment (start 100.965 132.715) (end 125.095 132.715) (width 0.25) (layer F.Cu) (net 12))
 (segment (start 125.73 130.175) (end 125.73 132.08) (width 0.25) (layer F.Cu) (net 12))
 (segment (start 100.965 115.57) (end 100.965 114.935) (width 0.25) (layer F.Cu) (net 12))
 (via (at 100.965 115.57) (size 0.6) (drill 0.4) (layers F.Cu B.Cu) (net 12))
 (segment (start 100.33 120.015) (end 100.33 116.205) (width 0.25) (layer B.Cu) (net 12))
 (segment (start 100.33 116.205) (end 100.965 115.57) (width 0.25) (layer B.Cu) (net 12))
 (segment (start 99.695 132.08) (end 99.695 120.65) (width 0.25) (layer F.Cu) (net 12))
 (segment (start 100.33 132.715) (end 99.695 132.08) (width 0.25) (layer F.Cu) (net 12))
 (segment (start 103.505 55.245) (end 101.6 55.245) (width 0.25) (layer F.Cu) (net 12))
 (segment (start 101.6 115.57) (end 103.505 115.57) (width 0.25) (layer F.Cu) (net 12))
 (segment (start 100.965 55.88) (end 100.965 114.935) (width 0.25) (layer F.Cu) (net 12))
 (segment (start 101.6 55.245) (end 100.965 55.88) (width 0.25) (layer F.Cu) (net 12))
 (via (at 100.33 121.285) (size 0.6) (drill 0.4) (layers F.Cu B.Cu) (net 13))
 (segment (start 100.965 119.38) (end 100.965 120.65) (width 0.25) (layer B.Cu) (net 13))
 (segment (start 100.965 120.65) (end 100.33 121.285) (width 0.25) (layer B.Cu) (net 13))
 (via (at 100.965 116.84) (size 0.6) (drill 0.4) (layers F.Cu B.Cu) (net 13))
 (segment (start 124.46 128.27) (end 124.46 131.445) (width 0.25) (layer F.Cu) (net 13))
 (segment (start 100.33 121.285) (end 100.33 131.445) (width 0.25) (layer F.Cu) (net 13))
 (segment (start 100.33 131.445) (end 100.965 132.08) (width 0.25) (layer F.Cu) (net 13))
 (segment (start 100.965 132.08) (end 101.6 132.08) (width 0.25) (layer F.Cu) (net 13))
 (segment (start 105.41 132.08) (end 101.6 132.08) (width 0.25) (layer F.Cu) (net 13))
 (segment (start 123.825 127.635) (end 124.46 128.27) (width 0.25) (layer F.Cu) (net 13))
 (segment (start 123.825 132.08) (end 105.41 132.08) (width 0.25) (layer F.Cu) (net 13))
 (segment (start 124.46 131.445) (end 123.825 132.08) (width 0.25) (layer F.Cu) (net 13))
 (segment (start 100.965 119.38) (end 100.965 116.84) (width 0.25) (layer B.Cu) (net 13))
 (segment (start 106.045 118.11) (end 106.045 117.475) (width 0.25) (layer F.Cu) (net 13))
 (segment (start 106.045 117.475) (end 105.41 116.84) (width 0.25) (layer F.Cu) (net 13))
 (segment (start 105.41 116.84) (end 100.965 116.84) (width 0.25) (layer F.Cu) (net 13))
 (segment (start 100.965 116.84) (end 100.33 116.205) (width 0.25) (layer F.Cu) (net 13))
 (segment (start 105.41 53.975) (end 106.045 53.34) (width 0.25) (layer F.Cu) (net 13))
 (segment (start 100.965 53.975) (end 105.41 53.975) (width 0.25) (layer F.Cu) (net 13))
 (segment (start 100.33 54.61) (end 100.965 53.975) (width 0.25) (layer F.Cu) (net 13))
 (segment (start 100.33 116.205) (end 100.33 54.61) (width 0.25) (layer F.Cu) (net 13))
 (segment (start 106.045 53.34) (end 106.045 52.705) (width 0.25) (layer F.Cu) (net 13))
 (segment (start 123.19 127.635) (end 123.825 127.635) (width 0.25) (layer F.Cu) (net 13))
 (via (at 99.06 120.015) (size 0.6) (drill 0.4) (layers F.Cu B.Cu) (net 11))
 (segment (start 99.06 120.015) (end 99.695 119.38) (width 0.25) (layer B.Cu) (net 11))
 (segment (start 101.6 114.3) (end 101.6 114.935) (width 0.25) (layer F.Cu) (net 11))
 (segment (start 99.695 115.57) (end 100.33 114.935) (width 0.25) (layer B.Cu) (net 11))
 (segment (start 99.695 115.57) (end 99.695 119.38) (width 0.25) (layer B.Cu) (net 11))
 (via (at 101.6 114.935) (size 0.6) (drill 0.4) (layers F.Cu B.Cu) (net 11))
 (segment (start 100.33 114.935) (end 101.6 114.935) (width 0.25) (layer B.Cu) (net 11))
 (segment (start 102.235 114.935) (end 102.87 114.3) (width 0.25) (layer F.Cu) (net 11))
 (segment (start 101.6 114.935) (end 102.235 114.935) (width 0.25) (layer F.Cu) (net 11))
 (segment (start 101.6 113.665) (end 101.6 114.3) (width 0.25) (layer F.Cu) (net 11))
 (segment (start 99.695 133.35) (end 100.33 133.35) (width 0.25) (layer F.Cu) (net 11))
 (segment (start 99.06 132.715) (end 99.695 133.35) (width 0.25) (layer F.Cu) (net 11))
 (segment (start 99.06 120.015) (end 99.06 132.715) (width 0.25) (layer F.Cu) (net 11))
 (segment (start 127 128.27) (end 127 132.715) (width 0.25) (layer F.Cu) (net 11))
 (segment (start 127 128.27) (end 126.365 127.635) (width 0.25) (layer F.Cu) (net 11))
 (segment (start 126.365 133.35) (end 100.33 133.35) (width 0.25) (layer F.Cu) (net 11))
 (segment (start 127 132.715) (end 126.365 133.35) (width 0.25) (layer F.Cu) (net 11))
 (segment (start 106.045 115.57) (end 106.045 114.935) (width 0.25) (layer F.Cu) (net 11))
 (segment (start 106.045 114.935) (end 105.41 114.3) (width 0.25) (layer F.Cu) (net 11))
 (segment (start 105.41 114.3) (end 102.87 114.3) (width 0.25) (layer F.Cu) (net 11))
 (segment (start 101.6 113.665) (end 101.6 57.15) (width 0.25) (layer F.Cu) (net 11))
 (segment (start 101.6 57.15) (end 102.235 56.515) (width 0.25) (layer F.Cu) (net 11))
 (segment (start 102.235 56.515) (end 105.41 56.515) (width 0.25) (layer F.Cu) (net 11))
 (segment (start 105.41 56.515) (end 106.045 55.88) (width 0.25) (layer F.Cu) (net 11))
 (segment (start 106.045 55.88) (end 106.045 55.245) (width 0.25) (layer F.Cu) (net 11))
 (segment (start 125.73 127.635) (end 126.365 127.635) (width 0.25) (layer F.Cu) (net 11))
 (segment (start 99.695 116.84) (end 100.965 118.11) (width 0.25) (layer F.Cu) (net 14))
 (segment (start 114.935 132.715) (end 118.11 132.715) (width 0.25) (layer B.Cu) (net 14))
 (segment (start 118.745 129.54) (end 119.38 128.905) (width 0.25) (layer B.Cu) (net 14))
 (segment (start 118.745 132.08) (end 118.745 129.54) (width 0.25) (layer B.Cu) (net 14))
 (segment (start 118.11 132.715) (end 118.745 132.08) (width 0.25) (layer B.Cu) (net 14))
 (segment (start 103.505 52.705) (end 100.33 52.705) (width 0.25) (layer F.Cu) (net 14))
 (segment (start 100.965 118.11) (end 103.505 118.11) (width 0.25) (layer F.Cu) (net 14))
 (segment (start 99.695 53.34) (end 99.695 116.84) (width 0.25) (layer F.Cu) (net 14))
 (segment (start 100.33 52.705) (end 99.695 53.34) (width 0.25) (layer F.Cu) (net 14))
 (segment (start 103.505 118.11) (end 104.14 118.11) (width 0.25) (layer B.Cu) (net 14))
 (segment (start 104.14 118.11) (end 104.775 118.745) (width 0.25) (layer B.Cu) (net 14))
 (segment (start 104.775 118.745) (end 104.775 132.08) (width 0.25) (layer B.Cu) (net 14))
 (segment (start 104.775 132.08) (end 105.41 132.715) (width 0.25) (layer B.Cu) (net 14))
 (segment (start 105.41 132.715) (end 114.935 132.715) (width 0.25) (layer B.Cu) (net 14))
 (segment (start 119.38 128.905) (end 122.555 128.905) (width 0.25) (layer B.Cu) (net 14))
 (segment (start 122.555 128.905) (end 123.19 129.54) (width 0.25) (layer B.Cu) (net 14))
 (segment (start 123.19 129.54) (end 123.19 130.175) (width 0.25) (layer B.Cu) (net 14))
 (segment (start 102.87 119.38) (end 100.965 119.38) (width 0.25) (layer F.Cu) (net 15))
 (segment (start 100.965 119.38) (end 100.33 118.745) (width 0.25) (layer F.Cu) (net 15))
 (segment (start 99.06 117.475) (end 100.33 118.745) (width 0.25) (layer F.Cu) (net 15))
 (segment (start 99.06 117.475) (end 99.06 52.07) (width 0.25) (layer F.Cu) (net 15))
 (segment (start 99.06 52.07) (end 99.695 51.435) (width 0.25) (layer F.Cu) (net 15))
 (segment (start 99.695 51.435) (end 105.41 51.435) (width 0.25) (layer F.Cu) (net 15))
 (segment (start 105.41 51.435) (end 106.045 50.8) (width 0.25) (layer F.Cu) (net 15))
 (segment (start 118.745 127.635) (end 118.11 128.27) (width 0.25) (layer B.Cu) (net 15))
 (segment (start 117.475 132.08) (end 114.3 132.08) (width 0.25) (layer B.Cu) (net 15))
 (segment (start 118.11 131.445) (end 117.475 132.08) (width 0.25) (layer B.Cu) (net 15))
 (segment (start 118.11 128.27) (end 118.11 131.445) (width 0.25) (layer B.Cu) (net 15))
 (segment (start 105.41 119.38) (end 102.87 119.38) (width 0.25) (layer F.Cu) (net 15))
 (segment (start 106.045 120.015) (end 105.41 119.38) (width 0.25) (layer F.Cu) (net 15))
 (segment (start 106.045 120.65) (end 106.045 120.015) (width 0.25) (layer F.Cu) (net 15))
 (segment (start 106.045 50.8) (end 106.045 50.165) (width 0.25) (layer F.Cu) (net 15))
 (segment (start 106.045 120.65) (end 106.045 131.445) (width 0.25) (layer B.Cu) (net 15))
 (segment (start 118.745 127.635) (end 120.65 127.635) (width 0.25) (layer B.Cu) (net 15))
 (segment (start 106.68 132.08) (end 114.3 132.08) (width 0.25) (layer B.Cu) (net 15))
 (segment (start 106.045 131.445) (end 106.68 132.08) (width 0.25) (layer B.Cu) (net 15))
 (segment (start 103.505 120.65) (end 100.965 120.65) (width 0.25) (layer F.Cu) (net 16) (status 400000))
 (segment (start 100.965 120.65) (end 100.33 120.015) (width 0.25) (layer F.Cu) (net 16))
 (segment (start 99.06 118.745) (end 100.33 120.015) (width 0.25) (layer F.Cu) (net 16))
 (via (at 99.06 118.745) (size 0.6) (drill 0.4) (layers F.Cu B.Cu) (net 16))
 (segment (start 103.505 50.165) (end 99.695 50.165) (width 0.25) (layer B.Cu) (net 16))
 (segment (start 99.06 50.8) (end 99.06 118.745) (width 0.25) (layer B.Cu) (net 16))
 (segment (start 99.695 50.165) (end 99.06 50.8) (width 0.25) (layer B.Cu) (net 16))
 (segment (start 102.87 120.65) (end 103.505 120.65) (width 0.25) (layer F.Cu) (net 16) (status C00000))
 (segment (start 120.65 130.175) (end 120.015 130.175) (width 0.25) (layer B.Cu) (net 16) (status C00000))
 (segment (start 120.015 130.175) (end 119.38 130.81) (width 0.25) (layer B.Cu) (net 16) (status 400000))
 (segment (start 118.745 133.35) (end 115.57 133.35) (width 0.25) (layer B.Cu) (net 16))
 (segment (start 119.38 132.715) (end 118.745 133.35) (width 0.25) (layer B.Cu) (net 16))
 (segment (start 119.38 130.81) (end 119.38 132.715) (width 0.25) (layer B.Cu) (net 16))
 (segment (start 103.505 132.715) (end 103.505 120.65) (width 0.25) (layer B.Cu) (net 16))
 (segment (start 115.57 133.35) (end 104.14 133.35) (width 0.25) (layer B.Cu) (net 16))
 (segment (start 104.14 133.35) (end 103.505 132.715) (width 0.25) (layer B.Cu) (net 16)))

